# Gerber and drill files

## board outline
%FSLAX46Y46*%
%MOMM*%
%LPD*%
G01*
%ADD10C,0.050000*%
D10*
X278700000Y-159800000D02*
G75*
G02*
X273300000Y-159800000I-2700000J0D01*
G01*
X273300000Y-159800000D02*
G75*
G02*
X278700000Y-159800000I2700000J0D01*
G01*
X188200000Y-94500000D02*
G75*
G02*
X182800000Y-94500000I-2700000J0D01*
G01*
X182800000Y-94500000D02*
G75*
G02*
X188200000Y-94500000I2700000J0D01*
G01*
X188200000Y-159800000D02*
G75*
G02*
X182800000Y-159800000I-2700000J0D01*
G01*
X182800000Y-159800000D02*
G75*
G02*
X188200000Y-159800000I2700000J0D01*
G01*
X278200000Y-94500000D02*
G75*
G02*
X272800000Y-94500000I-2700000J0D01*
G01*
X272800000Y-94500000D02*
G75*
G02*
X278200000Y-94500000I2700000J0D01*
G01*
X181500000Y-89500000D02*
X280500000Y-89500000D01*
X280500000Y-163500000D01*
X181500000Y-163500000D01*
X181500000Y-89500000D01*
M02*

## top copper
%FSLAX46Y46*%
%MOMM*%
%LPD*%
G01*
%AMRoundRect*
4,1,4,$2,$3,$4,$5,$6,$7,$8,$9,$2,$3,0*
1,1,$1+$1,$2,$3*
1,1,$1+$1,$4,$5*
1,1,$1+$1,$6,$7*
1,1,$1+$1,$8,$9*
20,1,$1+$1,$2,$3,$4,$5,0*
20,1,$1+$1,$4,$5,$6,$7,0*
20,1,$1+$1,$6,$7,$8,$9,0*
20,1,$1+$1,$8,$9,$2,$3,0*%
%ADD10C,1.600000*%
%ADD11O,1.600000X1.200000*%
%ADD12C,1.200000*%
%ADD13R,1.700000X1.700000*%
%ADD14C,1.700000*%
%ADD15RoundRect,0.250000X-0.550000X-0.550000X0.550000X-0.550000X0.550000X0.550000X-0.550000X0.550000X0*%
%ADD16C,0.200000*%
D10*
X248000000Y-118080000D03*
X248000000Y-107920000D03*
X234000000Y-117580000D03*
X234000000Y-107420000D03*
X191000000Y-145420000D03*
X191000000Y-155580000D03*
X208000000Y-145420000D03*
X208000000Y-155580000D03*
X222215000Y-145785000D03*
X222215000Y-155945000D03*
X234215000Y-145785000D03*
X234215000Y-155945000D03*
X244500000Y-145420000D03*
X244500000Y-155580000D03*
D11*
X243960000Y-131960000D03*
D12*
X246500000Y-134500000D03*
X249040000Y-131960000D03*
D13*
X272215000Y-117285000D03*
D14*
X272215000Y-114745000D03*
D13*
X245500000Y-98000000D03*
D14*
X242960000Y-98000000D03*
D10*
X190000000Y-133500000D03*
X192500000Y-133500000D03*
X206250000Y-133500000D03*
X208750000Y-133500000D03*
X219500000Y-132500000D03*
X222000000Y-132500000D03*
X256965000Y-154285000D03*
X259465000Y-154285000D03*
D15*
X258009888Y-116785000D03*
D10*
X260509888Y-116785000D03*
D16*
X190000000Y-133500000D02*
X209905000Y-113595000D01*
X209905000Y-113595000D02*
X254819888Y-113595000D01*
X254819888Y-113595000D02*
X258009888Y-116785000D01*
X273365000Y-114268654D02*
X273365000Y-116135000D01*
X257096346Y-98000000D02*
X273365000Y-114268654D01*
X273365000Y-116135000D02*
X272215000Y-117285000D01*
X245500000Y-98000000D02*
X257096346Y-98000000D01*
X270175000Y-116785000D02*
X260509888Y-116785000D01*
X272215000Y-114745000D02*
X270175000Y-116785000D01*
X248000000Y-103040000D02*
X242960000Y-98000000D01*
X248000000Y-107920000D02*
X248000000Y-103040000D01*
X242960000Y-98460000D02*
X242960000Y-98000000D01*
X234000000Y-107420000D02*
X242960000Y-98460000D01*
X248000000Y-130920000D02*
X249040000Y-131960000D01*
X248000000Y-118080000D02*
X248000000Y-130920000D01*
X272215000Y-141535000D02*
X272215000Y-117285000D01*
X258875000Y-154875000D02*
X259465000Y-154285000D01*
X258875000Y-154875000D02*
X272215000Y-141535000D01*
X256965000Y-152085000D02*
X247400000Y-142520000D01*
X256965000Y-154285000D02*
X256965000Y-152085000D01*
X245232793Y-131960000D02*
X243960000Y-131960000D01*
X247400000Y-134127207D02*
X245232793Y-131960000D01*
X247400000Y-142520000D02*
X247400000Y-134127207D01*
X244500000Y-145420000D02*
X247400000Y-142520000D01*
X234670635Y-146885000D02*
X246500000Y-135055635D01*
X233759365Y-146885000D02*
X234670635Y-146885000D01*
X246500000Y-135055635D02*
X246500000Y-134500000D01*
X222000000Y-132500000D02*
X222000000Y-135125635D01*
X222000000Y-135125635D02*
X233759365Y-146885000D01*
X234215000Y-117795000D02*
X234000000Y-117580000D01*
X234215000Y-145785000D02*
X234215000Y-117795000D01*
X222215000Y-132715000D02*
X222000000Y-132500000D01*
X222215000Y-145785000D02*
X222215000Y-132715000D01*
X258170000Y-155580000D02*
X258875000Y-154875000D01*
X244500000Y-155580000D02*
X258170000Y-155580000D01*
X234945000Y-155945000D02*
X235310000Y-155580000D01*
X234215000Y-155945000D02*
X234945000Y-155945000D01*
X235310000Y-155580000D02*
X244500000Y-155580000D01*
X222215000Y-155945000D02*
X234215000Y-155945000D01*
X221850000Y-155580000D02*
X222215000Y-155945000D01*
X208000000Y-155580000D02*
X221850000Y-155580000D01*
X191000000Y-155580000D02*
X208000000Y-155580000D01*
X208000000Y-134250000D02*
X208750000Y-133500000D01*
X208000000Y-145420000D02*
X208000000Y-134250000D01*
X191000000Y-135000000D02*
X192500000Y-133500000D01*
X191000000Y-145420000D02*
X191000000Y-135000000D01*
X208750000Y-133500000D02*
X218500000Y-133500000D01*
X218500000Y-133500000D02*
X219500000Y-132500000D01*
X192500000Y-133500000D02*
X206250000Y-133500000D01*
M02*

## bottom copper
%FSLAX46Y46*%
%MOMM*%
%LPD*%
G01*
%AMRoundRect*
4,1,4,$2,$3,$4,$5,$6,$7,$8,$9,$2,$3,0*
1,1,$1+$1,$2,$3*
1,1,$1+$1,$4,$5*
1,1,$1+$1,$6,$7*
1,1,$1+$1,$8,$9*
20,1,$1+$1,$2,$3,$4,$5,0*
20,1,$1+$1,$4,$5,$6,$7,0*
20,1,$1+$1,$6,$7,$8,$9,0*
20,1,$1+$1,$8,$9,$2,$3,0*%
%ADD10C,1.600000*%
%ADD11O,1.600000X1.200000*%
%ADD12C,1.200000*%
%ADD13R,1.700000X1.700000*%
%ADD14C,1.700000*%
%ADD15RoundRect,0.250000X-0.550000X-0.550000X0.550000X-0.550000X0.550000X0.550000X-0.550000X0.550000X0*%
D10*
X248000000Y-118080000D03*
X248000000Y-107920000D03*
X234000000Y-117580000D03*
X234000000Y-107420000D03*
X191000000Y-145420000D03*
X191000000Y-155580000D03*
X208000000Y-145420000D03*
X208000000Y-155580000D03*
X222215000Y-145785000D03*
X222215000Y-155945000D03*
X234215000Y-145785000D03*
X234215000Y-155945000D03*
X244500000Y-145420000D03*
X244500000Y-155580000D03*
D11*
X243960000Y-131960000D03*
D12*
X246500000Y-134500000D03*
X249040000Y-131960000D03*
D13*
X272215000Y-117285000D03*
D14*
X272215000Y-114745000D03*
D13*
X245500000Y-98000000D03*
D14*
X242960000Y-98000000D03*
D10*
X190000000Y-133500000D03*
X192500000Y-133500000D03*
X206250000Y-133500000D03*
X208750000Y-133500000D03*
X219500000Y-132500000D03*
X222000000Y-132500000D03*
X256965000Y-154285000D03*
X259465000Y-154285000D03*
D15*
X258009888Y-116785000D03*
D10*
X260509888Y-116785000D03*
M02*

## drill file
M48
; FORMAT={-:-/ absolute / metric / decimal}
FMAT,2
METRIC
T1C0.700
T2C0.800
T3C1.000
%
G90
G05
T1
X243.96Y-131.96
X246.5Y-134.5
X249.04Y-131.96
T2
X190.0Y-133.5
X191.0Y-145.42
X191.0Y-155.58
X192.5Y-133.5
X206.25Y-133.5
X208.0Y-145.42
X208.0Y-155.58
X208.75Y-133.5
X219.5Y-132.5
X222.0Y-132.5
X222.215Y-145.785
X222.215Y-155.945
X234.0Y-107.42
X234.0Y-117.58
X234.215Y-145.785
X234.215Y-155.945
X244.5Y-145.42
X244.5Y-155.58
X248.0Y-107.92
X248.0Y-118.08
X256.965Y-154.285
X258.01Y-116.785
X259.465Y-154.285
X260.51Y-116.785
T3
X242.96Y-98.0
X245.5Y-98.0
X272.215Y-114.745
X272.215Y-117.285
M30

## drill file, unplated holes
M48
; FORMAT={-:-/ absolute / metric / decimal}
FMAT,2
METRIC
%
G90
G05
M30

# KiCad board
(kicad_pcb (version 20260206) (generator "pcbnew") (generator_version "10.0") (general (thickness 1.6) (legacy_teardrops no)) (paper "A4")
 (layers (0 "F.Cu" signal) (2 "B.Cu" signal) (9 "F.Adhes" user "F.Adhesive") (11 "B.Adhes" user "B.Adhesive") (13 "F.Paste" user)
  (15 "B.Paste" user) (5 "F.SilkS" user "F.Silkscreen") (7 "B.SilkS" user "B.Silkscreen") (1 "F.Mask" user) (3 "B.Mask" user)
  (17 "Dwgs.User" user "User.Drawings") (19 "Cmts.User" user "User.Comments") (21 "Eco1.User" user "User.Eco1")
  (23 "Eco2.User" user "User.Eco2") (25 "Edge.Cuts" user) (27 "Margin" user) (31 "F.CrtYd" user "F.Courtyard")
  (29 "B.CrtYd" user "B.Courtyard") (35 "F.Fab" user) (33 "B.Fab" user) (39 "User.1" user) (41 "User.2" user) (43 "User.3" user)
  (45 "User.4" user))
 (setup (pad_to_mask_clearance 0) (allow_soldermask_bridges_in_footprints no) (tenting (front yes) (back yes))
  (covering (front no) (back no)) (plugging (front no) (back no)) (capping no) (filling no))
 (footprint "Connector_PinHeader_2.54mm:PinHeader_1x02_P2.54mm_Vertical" (layer "F.Cu") (at 272 118.92 180)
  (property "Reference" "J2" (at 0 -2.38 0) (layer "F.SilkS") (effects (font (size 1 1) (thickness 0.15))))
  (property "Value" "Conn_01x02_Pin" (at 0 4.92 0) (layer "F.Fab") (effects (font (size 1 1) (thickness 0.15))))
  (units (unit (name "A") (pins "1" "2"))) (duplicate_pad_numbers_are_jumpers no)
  (pad "1" thru_hole rect (at 0 0 180) (size 1.7 1.7) (drill 1) (layers "*.Cu" "*.Mask") (remove_unused_layers no) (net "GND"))
  (pad "2" thru_hole circle (at 0 2.54 180) (size 1.7 1.7) (drill 1) (layers "*.Cu" "*.Mask") (remove_unused_layers no)
   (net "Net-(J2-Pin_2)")))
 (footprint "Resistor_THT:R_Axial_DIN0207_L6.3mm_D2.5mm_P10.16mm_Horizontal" (layer "F.Cu") (at 222 147.42 -90)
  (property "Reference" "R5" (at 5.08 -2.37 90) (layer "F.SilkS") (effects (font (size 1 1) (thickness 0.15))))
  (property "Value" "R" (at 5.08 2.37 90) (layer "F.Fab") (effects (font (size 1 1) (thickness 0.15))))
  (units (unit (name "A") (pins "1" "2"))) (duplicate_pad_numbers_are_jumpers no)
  (pad "1" thru_hole circle (at 0 0 270) (size 1.6 1.6) (drill 0.8) (layers "*.Cu" "*.Mask") (remove_unused_layers no) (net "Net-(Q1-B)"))
  (pad "2" thru_hole circle (at 10.16 0 270) (size 1.6 1.6) (drill 0.8) (layers "*.Cu" "*.Mask") (remove_unused_layers no) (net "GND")))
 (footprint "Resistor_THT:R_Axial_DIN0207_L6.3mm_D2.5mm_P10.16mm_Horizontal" (layer "F.Cu") (at 234 147.42 -90)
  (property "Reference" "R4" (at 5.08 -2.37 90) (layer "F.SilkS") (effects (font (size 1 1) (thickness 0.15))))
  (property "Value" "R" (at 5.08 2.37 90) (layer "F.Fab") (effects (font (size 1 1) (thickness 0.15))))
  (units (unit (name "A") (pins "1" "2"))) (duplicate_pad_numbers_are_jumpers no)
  (pad "1" thru_hole circle (at 0 0 270) (size 1.6 1.6) (drill 0.8) (layers "*.Cu" "*.Mask") (remove_unused_layers no) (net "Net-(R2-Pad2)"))
  (pad "2" thru_hole circle (at 10.16 0 270) (size 1.6 1.6) (drill 0.8) (layers "*.Cu" "*.Mask") (remove_unused_layers no) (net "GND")))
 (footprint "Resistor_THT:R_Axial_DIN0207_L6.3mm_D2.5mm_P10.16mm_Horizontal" (layer "F.Cu") (at 247.785 109.555 -90)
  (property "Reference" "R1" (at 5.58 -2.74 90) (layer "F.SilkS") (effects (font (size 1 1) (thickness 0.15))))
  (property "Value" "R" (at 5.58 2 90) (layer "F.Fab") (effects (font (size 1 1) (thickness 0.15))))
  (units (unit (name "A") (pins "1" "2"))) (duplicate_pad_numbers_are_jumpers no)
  (pad "1" thru_hole circle (at 0 0 270) (size 1.6 1.6) (drill 0.8) (layers "*.Cu" "*.Mask") (remove_unused_layers no)
   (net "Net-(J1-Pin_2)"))
  (pad "2" thru_hole circle (at 10.16 0 270) (size 1.6 1.6) (drill 0.8) (layers "*.Cu" "*.Mask") (remove_unused_layers no)
   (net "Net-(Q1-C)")))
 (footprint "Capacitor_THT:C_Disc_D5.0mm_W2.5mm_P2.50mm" (layer "F.Cu") (at 256.75 155.92)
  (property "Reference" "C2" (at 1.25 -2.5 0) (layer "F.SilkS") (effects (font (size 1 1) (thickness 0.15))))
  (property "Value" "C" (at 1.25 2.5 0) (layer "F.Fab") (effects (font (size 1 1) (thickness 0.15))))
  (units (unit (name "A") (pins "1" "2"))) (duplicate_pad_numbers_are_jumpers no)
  (pad "1" thru_hole circle (at 0 0) (size 1.6 1.6) (drill 0.8) (layers "*.Cu" "*.Mask") (remove_unused_layers no) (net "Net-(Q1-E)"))
  (pad "2" thru_hole circle (at 2.5 0) (size 1.6 1.6) (drill 0.8) (layers "*.Cu" "*.Mask") (remove_unused_layers no) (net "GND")))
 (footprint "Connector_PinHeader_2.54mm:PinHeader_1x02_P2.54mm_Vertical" (layer "F.Cu") (at 245.285 99.635 -90)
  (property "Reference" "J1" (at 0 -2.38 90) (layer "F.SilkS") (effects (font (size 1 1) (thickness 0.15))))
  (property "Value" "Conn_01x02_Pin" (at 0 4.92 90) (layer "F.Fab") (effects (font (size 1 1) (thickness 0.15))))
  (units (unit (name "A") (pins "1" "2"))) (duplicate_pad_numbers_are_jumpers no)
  (pad "1" thru_hole rect (at 0 0 270) (size 1.7 1.7) (drill 1) (layers "*.Cu" "*.Mask") (remove_unused_layers no) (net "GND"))
  (pad "2" thru_hole circle (at 0 2.54 270) (size 1.7 1.7) (drill 1) (layers "*.Cu" "*.Mask") (remove_unused_layers no)
   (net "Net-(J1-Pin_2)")))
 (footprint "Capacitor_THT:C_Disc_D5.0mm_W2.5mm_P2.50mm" (layer "F.Cu") (at 219.285 134.135)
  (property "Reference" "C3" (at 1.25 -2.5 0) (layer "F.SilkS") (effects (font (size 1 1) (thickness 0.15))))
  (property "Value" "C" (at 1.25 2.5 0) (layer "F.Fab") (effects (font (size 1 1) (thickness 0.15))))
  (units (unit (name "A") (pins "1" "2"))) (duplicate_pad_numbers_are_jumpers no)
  (pad "1" thru_hole circle (at 0 0) (size 1.6 1.6) (drill 0.8) (layers "*.Cu" "*.Mask") (remove_unused_layers no) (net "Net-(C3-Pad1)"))
  (pad "2" thru_hole circle (at 2.5 0) (size 1.6 1.6) (drill 0.8) (layers "*.Cu" "*.Mask") (remove_unused_layers no) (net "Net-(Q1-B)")))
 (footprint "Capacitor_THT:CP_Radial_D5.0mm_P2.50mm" (layer "F.Cu") (at 257.794888 118.42)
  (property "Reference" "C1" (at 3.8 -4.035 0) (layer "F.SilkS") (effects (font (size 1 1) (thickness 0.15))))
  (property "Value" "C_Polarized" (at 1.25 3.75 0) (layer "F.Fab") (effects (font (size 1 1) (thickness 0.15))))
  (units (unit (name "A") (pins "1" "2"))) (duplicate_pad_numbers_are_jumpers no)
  (pad "1" thru_hole roundrect (at 0 0) (size 1.6 1.6) (drill 0.8) (layers "*.Cu" "*.Mask") (remove_unused_layers no)
   (roundrect_rratio 0.15625) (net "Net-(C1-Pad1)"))
  (pad "2" thru_hole circle (at 2.5 0) (size 1.6 1.6) (drill 0.8) (layers "*.Cu" "*.Mask") (remove_unused_layers no) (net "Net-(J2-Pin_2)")))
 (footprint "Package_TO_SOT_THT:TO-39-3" (layer "F.Cu") (at 243.745 133.595)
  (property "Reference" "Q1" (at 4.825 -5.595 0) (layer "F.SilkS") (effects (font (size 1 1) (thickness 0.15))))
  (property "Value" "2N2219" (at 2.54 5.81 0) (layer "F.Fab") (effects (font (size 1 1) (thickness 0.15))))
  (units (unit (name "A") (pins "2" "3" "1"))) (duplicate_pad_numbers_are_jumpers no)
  (pad "1" thru_hole oval (at 0 0) (size 1.6 1.2) (drill 0.7) (layers "*.Cu" "*.Mask") (remove_unused_layers no) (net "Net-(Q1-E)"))
  (pad "2" thru_hole circle (at 2.54 2.54) (size 1.2 1.2) (drill 0.7) (layers "*.Cu" "*.Mask") (remove_unused_layers no) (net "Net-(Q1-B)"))
  (pad "3" thru_hole circle (at 5.08 0) (size 1.2 1.2) (drill 0.7) (layers "*.Cu" "*.Mask") (remove_unused_layers no) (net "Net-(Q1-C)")))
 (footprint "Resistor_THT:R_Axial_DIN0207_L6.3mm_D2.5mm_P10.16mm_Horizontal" (layer "F.Cu") (at 207.785 147.055 -90)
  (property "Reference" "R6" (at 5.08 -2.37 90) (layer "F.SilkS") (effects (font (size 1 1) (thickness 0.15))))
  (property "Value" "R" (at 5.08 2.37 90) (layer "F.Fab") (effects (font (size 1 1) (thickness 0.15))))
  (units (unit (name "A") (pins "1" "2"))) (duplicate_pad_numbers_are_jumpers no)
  (pad "1" thru_hole circle (at 0 0 270) (size 1.6 1.6) (drill 0.8) (layers "*.Cu" "*.Mask") (remove_unused_layers no) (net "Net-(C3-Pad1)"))
  (pad "2" thru_hole circle (at 10.16 0 270) (size 1.6 1.6) (drill 0.8) (layers "*.Cu" "*.Mask") (remove_unused_layers no) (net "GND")))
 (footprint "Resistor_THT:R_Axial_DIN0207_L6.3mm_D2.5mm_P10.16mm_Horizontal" (layer "F.Cu") (at 233.785 109.055 -90)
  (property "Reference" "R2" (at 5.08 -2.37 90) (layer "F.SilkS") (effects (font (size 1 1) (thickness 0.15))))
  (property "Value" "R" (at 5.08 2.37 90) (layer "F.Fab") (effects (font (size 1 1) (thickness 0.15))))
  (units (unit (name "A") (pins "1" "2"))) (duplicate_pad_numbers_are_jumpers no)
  (pad "1" thru_hole circle (at 0 0 270) (size 1.6 1.6) (drill 0.8) (layers "*.Cu" "*.Mask") (remove_unused_layers no)
   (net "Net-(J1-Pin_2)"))
  (pad "2" thru_hole circle (at 10.16 0 270) (size 1.6 1.6) (drill 0.8) (layers "*.Cu" "*.Mask") (remove_unused_layers no)
   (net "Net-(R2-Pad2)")))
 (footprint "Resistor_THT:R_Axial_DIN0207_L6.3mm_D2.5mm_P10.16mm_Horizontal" (layer "F.Cu") (at 190.785 147.055 -90)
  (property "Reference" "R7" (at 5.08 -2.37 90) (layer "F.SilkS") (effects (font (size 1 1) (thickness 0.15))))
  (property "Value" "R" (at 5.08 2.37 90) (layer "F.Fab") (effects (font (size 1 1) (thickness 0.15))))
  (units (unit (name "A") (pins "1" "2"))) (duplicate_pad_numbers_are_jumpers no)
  (pad "1" thru_hole circle (at 0 0 270) (size 1.6 1.6) (drill 0.8) (layers "*.Cu" "*.Mask") (remove_unused_layers no) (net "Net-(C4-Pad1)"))
  (pad "2" thru_hole circle (at 10.16 0 270) (size 1.6 1.6) (drill 0.8) (layers "*.Cu" "*.Mask") (remove_unused_layers no) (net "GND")))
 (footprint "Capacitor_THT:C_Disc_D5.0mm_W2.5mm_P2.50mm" (layer "F.Cu") (at 189.785 135.135)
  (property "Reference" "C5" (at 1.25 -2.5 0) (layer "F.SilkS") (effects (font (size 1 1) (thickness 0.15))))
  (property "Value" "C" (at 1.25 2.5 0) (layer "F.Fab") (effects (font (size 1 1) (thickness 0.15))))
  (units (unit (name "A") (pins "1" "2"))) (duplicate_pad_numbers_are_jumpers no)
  (pad "1" thru_hole circle (at 0 0) (size 1.6 1.6) (drill 0.8) (layers "*.Cu" "*.Mask") (remove_unused_layers no) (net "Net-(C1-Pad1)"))
  (pad "2" thru_hole circle (at 2.5 0) (size 1.6 1.6) (drill 0.8) (layers "*.Cu" "*.Mask") (remove_unused_layers no) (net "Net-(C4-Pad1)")))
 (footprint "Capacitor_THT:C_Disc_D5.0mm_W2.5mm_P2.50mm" (layer "F.Cu") (at 206.035 135.135)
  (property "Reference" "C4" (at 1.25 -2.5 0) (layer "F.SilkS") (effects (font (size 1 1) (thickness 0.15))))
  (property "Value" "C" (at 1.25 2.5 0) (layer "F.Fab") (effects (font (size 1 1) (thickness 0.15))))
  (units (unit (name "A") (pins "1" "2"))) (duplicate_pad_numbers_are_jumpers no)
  (pad "1" thru_hole circle (at 0 0) (size 1.6 1.6) (drill 0.8) (layers "*.Cu" "*.Mask") (remove_unused_layers no) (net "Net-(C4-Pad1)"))
  (pad "2" thru_hole circle (at 2.5 0) (size 1.6 1.6) (drill 0.8) (layers "*.Cu" "*.Mask") (remove_unused_layers no) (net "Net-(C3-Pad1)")))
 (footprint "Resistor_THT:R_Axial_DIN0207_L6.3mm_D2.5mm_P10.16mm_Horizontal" (layer "F.Cu") (at 244.285 147.055 -90)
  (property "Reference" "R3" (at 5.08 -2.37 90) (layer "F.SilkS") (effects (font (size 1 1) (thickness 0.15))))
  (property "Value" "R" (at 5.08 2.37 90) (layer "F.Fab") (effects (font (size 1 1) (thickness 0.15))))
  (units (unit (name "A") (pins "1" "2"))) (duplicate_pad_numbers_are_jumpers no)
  (pad "1" thru_hole circle (at 0 0 270) (size 1.6 1.6) (drill 0.8) (layers "*.Cu" "*.Mask") (remove_unused_layers no) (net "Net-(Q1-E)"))
  (pad "2" thru_hole circle (at 10.16 0 270) (size 1.6 1.6) (drill 0.8) (layers "*.Cu" "*.Mask") (remove_unused_layers no) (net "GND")))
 (gr_rect (start 181.285 91.135) (end 280.285 165.135) (stroke (width 0.05) (type default)) (fill no) (layer "Edge.Cuts"))
 (gr_circle (center 185.285 96.135) (end 187.985 96.135) (stroke (width 0.05) (type solid)) (fill no) (layer "Edge.Cuts"))
 (gr_circle (center 185.285 161.435) (end 187.985 161.435) (stroke (width 0.05) (type solid)) (fill no) (layer "Edge.Cuts"))
 (gr_circle (center 275.285 96.135) (end 277.985 96.135) (stroke (width 0.05) (type solid)) (fill no) (layer "Edge.Cuts"))
 (gr_circle (center 275.785 161.435) (end 278.485 161.435) (stroke (width 0.05) (type solid)) (fill no) (layer "Edge.Cuts"))
 (segment (start 272 143.17) (end 272 118.92) (width 0.2) (layer "F.Cu") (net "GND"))
 (segment (start 258.66 156.51) (end 272 143.17) (width 0.2) (layer "F.Cu") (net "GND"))
 (segment (start 256.881346 99.635) (end 273.15 115.903654) (width 0.2) (layer "F.Cu") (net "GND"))
 (segment (start 190.785 157.215) (end 207.785 157.215) (width 0.2) (layer "F.Cu") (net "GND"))
 (segment (start 258.66 156.51) (end 259.25 155.92) (width 0.2) (layer "F.Cu") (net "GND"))
 (segment (start 222 157.58) (end 234 157.58) (width 0.2) (layer "F.Cu") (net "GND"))
 (segment (start 221.635 157.215) (end 222 157.58) (width 0.2) (layer "F.Cu") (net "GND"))
 (segment (start 273.15 117.77) (end 272 118.92) (width 0.2) (layer "F.Cu") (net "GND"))
 (segment (start 234.73 157.58) (end 235.095 157.215) (width 0.2) (layer "F.Cu") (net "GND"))
 (segment (start 245.285 99.635) (end 256.881346 99.635) (width 0.2) (layer "F.Cu") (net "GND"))
 (segment (start 273.15 115.903654) (end 273.15 117.77) (width 0.2) (layer "F.Cu") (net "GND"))
 (segment (start 234 157.58) (end 234.73 157.58) (width 0.2) (layer "F.Cu") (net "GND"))
 (segment (start 244.285 157.215) (end 257.955 157.215) (width 0.2) (layer "F.Cu") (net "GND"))
 (segment (start 235.095 157.215) (end 244.285 157.215) (width 0.2) (layer "F.Cu") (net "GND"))
 (segment (start 207.785 157.215) (end 221.635 157.215) (width 0.2) (layer "F.Cu") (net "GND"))
 (segment (start 257.955 157.215) (end 258.66 156.51) (width 0.2) (layer "F.Cu") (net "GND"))
 (segment (start 272 116.38) (end 269.96 118.42) (width 0.2) (layer "F.Cu") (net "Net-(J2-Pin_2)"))
 (segment (start 269.96 118.42) (end 260.294888 118.42) (width 0.2) (layer "F.Cu") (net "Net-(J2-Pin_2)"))
 (segment (start 221.785 134.135) (end 221.785 136.760635) (width 0.2) (layer "F.Cu") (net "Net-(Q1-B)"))
 (segment (start 233.544365 148.52) (end 234.455635 148.52) (width 0.2) (layer "F.Cu") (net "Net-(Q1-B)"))
 (segment (start 222 134.35) (end 221.785 134.135) (width 0.2) (layer "F.Cu") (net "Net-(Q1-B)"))
 (segment (start 222 147.42) (end 222 134.35) (width 0.2) (layer "F.Cu") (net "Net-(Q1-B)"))
 (segment (start 246.285 136.690635) (end 246.285 136.135) (width 0.2) (layer "F.Cu") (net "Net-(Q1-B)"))
 (segment (start 234.455635 148.52) (end 246.285 136.690635) (width 0.2) (layer "F.Cu") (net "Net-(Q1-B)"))
 (segment (start 221.785 136.760635) (end 233.544365 148.52) (width 0.2) (layer "F.Cu") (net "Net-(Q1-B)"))
 (segment (start 234 119.43) (end 233.785 119.215) (width 0.2) (layer "F.Cu") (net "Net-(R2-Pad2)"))
 (segment (start 234 147.42) (end 234 119.43) (width 0.2) (layer "F.Cu") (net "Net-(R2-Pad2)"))
 (segment (start 247.785 109.555) (end 247.785 104.675) (width 0.2) (layer "F.Cu") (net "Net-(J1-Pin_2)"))
 (segment (start 242.745 100.095) (end 242.745 99.635) (width 0.2) (layer "F.Cu") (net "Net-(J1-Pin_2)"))
 (segment (start 233.785 109.055) (end 242.745 100.095) (width 0.2) (layer "F.Cu") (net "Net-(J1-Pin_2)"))
 (segment (start 247.785 104.675) (end 242.745 99.635) (width 0.2) (layer "F.Cu") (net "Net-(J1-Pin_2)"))
 (segment (start 247.785 132.555) (end 248.825 133.595) (width 0.2) (layer "F.Cu") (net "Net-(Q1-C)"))
 (segment (start 247.785 119.715) (end 247.785 132.555) (width 0.2) (layer "F.Cu") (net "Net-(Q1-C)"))
 (segment (start 244.285 147.055) (end 247.185 144.155) (width 0.2) (layer "F.Cu") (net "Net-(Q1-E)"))
 (segment (start 245.017793 133.595) (end 243.745 133.595) (width 0.2) (layer "F.Cu") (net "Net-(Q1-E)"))
 (segment (start 247.185 135.762207) (end 245.017793 133.595) (width 0.2) (layer "F.Cu") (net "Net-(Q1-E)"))
 (segment (start 256.75 155.92) (end 256.75 153.72) (width 0.2) (layer "F.Cu") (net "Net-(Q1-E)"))
 (segment (start 247.185 144.155) (end 247.185 135.762207) (width 0.2) (layer "F.Cu") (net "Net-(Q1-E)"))
 (segment (start 256.75 153.72) (end 247.185 144.155) (width 0.2) (layer "F.Cu") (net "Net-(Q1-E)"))
 (segment (start 207.785 135.885) (end 208.535 135.135) (width 0.2) (layer "F.Cu") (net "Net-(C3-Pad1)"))
 (segment (start 208.535 135.135) (end 218.285 135.135) (width 0.2) (layer "F.Cu") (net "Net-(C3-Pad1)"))
 (segment (start 218.285 135.135) (end 219.285 134.135) (width 0.2) (layer "F.Cu") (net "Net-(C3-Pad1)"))
 (segment (start 207.785 147.055) (end 207.785 135.885) (width 0.2) (layer "F.Cu") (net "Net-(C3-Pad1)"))
 (segment (start 254.604888 115.23) (end 257.794888 118.42) (width 0.2) (layer "F.Cu") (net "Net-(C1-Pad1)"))
 (segment (start 189.785 135.135) (end 209.69 115.23) (width 0.2) (layer "F.Cu") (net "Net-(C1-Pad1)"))
 (segment (start 209.69 115.23) (end 254.604888 115.23) (width 0.2) (layer "F.Cu") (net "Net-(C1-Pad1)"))
 (segment (start 190.785 147.055) (end 190.785 136.635) (width 0.2) (layer "F.Cu") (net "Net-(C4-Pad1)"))
 (segment (start 192.285 135.135) (end 206.035 135.135) (width 0.2) (layer "F.Cu") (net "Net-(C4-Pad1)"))
 (segment (start 190.785 136.635) (end 192.285 135.135) (width 0.2) (layer "F.Cu") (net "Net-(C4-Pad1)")))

